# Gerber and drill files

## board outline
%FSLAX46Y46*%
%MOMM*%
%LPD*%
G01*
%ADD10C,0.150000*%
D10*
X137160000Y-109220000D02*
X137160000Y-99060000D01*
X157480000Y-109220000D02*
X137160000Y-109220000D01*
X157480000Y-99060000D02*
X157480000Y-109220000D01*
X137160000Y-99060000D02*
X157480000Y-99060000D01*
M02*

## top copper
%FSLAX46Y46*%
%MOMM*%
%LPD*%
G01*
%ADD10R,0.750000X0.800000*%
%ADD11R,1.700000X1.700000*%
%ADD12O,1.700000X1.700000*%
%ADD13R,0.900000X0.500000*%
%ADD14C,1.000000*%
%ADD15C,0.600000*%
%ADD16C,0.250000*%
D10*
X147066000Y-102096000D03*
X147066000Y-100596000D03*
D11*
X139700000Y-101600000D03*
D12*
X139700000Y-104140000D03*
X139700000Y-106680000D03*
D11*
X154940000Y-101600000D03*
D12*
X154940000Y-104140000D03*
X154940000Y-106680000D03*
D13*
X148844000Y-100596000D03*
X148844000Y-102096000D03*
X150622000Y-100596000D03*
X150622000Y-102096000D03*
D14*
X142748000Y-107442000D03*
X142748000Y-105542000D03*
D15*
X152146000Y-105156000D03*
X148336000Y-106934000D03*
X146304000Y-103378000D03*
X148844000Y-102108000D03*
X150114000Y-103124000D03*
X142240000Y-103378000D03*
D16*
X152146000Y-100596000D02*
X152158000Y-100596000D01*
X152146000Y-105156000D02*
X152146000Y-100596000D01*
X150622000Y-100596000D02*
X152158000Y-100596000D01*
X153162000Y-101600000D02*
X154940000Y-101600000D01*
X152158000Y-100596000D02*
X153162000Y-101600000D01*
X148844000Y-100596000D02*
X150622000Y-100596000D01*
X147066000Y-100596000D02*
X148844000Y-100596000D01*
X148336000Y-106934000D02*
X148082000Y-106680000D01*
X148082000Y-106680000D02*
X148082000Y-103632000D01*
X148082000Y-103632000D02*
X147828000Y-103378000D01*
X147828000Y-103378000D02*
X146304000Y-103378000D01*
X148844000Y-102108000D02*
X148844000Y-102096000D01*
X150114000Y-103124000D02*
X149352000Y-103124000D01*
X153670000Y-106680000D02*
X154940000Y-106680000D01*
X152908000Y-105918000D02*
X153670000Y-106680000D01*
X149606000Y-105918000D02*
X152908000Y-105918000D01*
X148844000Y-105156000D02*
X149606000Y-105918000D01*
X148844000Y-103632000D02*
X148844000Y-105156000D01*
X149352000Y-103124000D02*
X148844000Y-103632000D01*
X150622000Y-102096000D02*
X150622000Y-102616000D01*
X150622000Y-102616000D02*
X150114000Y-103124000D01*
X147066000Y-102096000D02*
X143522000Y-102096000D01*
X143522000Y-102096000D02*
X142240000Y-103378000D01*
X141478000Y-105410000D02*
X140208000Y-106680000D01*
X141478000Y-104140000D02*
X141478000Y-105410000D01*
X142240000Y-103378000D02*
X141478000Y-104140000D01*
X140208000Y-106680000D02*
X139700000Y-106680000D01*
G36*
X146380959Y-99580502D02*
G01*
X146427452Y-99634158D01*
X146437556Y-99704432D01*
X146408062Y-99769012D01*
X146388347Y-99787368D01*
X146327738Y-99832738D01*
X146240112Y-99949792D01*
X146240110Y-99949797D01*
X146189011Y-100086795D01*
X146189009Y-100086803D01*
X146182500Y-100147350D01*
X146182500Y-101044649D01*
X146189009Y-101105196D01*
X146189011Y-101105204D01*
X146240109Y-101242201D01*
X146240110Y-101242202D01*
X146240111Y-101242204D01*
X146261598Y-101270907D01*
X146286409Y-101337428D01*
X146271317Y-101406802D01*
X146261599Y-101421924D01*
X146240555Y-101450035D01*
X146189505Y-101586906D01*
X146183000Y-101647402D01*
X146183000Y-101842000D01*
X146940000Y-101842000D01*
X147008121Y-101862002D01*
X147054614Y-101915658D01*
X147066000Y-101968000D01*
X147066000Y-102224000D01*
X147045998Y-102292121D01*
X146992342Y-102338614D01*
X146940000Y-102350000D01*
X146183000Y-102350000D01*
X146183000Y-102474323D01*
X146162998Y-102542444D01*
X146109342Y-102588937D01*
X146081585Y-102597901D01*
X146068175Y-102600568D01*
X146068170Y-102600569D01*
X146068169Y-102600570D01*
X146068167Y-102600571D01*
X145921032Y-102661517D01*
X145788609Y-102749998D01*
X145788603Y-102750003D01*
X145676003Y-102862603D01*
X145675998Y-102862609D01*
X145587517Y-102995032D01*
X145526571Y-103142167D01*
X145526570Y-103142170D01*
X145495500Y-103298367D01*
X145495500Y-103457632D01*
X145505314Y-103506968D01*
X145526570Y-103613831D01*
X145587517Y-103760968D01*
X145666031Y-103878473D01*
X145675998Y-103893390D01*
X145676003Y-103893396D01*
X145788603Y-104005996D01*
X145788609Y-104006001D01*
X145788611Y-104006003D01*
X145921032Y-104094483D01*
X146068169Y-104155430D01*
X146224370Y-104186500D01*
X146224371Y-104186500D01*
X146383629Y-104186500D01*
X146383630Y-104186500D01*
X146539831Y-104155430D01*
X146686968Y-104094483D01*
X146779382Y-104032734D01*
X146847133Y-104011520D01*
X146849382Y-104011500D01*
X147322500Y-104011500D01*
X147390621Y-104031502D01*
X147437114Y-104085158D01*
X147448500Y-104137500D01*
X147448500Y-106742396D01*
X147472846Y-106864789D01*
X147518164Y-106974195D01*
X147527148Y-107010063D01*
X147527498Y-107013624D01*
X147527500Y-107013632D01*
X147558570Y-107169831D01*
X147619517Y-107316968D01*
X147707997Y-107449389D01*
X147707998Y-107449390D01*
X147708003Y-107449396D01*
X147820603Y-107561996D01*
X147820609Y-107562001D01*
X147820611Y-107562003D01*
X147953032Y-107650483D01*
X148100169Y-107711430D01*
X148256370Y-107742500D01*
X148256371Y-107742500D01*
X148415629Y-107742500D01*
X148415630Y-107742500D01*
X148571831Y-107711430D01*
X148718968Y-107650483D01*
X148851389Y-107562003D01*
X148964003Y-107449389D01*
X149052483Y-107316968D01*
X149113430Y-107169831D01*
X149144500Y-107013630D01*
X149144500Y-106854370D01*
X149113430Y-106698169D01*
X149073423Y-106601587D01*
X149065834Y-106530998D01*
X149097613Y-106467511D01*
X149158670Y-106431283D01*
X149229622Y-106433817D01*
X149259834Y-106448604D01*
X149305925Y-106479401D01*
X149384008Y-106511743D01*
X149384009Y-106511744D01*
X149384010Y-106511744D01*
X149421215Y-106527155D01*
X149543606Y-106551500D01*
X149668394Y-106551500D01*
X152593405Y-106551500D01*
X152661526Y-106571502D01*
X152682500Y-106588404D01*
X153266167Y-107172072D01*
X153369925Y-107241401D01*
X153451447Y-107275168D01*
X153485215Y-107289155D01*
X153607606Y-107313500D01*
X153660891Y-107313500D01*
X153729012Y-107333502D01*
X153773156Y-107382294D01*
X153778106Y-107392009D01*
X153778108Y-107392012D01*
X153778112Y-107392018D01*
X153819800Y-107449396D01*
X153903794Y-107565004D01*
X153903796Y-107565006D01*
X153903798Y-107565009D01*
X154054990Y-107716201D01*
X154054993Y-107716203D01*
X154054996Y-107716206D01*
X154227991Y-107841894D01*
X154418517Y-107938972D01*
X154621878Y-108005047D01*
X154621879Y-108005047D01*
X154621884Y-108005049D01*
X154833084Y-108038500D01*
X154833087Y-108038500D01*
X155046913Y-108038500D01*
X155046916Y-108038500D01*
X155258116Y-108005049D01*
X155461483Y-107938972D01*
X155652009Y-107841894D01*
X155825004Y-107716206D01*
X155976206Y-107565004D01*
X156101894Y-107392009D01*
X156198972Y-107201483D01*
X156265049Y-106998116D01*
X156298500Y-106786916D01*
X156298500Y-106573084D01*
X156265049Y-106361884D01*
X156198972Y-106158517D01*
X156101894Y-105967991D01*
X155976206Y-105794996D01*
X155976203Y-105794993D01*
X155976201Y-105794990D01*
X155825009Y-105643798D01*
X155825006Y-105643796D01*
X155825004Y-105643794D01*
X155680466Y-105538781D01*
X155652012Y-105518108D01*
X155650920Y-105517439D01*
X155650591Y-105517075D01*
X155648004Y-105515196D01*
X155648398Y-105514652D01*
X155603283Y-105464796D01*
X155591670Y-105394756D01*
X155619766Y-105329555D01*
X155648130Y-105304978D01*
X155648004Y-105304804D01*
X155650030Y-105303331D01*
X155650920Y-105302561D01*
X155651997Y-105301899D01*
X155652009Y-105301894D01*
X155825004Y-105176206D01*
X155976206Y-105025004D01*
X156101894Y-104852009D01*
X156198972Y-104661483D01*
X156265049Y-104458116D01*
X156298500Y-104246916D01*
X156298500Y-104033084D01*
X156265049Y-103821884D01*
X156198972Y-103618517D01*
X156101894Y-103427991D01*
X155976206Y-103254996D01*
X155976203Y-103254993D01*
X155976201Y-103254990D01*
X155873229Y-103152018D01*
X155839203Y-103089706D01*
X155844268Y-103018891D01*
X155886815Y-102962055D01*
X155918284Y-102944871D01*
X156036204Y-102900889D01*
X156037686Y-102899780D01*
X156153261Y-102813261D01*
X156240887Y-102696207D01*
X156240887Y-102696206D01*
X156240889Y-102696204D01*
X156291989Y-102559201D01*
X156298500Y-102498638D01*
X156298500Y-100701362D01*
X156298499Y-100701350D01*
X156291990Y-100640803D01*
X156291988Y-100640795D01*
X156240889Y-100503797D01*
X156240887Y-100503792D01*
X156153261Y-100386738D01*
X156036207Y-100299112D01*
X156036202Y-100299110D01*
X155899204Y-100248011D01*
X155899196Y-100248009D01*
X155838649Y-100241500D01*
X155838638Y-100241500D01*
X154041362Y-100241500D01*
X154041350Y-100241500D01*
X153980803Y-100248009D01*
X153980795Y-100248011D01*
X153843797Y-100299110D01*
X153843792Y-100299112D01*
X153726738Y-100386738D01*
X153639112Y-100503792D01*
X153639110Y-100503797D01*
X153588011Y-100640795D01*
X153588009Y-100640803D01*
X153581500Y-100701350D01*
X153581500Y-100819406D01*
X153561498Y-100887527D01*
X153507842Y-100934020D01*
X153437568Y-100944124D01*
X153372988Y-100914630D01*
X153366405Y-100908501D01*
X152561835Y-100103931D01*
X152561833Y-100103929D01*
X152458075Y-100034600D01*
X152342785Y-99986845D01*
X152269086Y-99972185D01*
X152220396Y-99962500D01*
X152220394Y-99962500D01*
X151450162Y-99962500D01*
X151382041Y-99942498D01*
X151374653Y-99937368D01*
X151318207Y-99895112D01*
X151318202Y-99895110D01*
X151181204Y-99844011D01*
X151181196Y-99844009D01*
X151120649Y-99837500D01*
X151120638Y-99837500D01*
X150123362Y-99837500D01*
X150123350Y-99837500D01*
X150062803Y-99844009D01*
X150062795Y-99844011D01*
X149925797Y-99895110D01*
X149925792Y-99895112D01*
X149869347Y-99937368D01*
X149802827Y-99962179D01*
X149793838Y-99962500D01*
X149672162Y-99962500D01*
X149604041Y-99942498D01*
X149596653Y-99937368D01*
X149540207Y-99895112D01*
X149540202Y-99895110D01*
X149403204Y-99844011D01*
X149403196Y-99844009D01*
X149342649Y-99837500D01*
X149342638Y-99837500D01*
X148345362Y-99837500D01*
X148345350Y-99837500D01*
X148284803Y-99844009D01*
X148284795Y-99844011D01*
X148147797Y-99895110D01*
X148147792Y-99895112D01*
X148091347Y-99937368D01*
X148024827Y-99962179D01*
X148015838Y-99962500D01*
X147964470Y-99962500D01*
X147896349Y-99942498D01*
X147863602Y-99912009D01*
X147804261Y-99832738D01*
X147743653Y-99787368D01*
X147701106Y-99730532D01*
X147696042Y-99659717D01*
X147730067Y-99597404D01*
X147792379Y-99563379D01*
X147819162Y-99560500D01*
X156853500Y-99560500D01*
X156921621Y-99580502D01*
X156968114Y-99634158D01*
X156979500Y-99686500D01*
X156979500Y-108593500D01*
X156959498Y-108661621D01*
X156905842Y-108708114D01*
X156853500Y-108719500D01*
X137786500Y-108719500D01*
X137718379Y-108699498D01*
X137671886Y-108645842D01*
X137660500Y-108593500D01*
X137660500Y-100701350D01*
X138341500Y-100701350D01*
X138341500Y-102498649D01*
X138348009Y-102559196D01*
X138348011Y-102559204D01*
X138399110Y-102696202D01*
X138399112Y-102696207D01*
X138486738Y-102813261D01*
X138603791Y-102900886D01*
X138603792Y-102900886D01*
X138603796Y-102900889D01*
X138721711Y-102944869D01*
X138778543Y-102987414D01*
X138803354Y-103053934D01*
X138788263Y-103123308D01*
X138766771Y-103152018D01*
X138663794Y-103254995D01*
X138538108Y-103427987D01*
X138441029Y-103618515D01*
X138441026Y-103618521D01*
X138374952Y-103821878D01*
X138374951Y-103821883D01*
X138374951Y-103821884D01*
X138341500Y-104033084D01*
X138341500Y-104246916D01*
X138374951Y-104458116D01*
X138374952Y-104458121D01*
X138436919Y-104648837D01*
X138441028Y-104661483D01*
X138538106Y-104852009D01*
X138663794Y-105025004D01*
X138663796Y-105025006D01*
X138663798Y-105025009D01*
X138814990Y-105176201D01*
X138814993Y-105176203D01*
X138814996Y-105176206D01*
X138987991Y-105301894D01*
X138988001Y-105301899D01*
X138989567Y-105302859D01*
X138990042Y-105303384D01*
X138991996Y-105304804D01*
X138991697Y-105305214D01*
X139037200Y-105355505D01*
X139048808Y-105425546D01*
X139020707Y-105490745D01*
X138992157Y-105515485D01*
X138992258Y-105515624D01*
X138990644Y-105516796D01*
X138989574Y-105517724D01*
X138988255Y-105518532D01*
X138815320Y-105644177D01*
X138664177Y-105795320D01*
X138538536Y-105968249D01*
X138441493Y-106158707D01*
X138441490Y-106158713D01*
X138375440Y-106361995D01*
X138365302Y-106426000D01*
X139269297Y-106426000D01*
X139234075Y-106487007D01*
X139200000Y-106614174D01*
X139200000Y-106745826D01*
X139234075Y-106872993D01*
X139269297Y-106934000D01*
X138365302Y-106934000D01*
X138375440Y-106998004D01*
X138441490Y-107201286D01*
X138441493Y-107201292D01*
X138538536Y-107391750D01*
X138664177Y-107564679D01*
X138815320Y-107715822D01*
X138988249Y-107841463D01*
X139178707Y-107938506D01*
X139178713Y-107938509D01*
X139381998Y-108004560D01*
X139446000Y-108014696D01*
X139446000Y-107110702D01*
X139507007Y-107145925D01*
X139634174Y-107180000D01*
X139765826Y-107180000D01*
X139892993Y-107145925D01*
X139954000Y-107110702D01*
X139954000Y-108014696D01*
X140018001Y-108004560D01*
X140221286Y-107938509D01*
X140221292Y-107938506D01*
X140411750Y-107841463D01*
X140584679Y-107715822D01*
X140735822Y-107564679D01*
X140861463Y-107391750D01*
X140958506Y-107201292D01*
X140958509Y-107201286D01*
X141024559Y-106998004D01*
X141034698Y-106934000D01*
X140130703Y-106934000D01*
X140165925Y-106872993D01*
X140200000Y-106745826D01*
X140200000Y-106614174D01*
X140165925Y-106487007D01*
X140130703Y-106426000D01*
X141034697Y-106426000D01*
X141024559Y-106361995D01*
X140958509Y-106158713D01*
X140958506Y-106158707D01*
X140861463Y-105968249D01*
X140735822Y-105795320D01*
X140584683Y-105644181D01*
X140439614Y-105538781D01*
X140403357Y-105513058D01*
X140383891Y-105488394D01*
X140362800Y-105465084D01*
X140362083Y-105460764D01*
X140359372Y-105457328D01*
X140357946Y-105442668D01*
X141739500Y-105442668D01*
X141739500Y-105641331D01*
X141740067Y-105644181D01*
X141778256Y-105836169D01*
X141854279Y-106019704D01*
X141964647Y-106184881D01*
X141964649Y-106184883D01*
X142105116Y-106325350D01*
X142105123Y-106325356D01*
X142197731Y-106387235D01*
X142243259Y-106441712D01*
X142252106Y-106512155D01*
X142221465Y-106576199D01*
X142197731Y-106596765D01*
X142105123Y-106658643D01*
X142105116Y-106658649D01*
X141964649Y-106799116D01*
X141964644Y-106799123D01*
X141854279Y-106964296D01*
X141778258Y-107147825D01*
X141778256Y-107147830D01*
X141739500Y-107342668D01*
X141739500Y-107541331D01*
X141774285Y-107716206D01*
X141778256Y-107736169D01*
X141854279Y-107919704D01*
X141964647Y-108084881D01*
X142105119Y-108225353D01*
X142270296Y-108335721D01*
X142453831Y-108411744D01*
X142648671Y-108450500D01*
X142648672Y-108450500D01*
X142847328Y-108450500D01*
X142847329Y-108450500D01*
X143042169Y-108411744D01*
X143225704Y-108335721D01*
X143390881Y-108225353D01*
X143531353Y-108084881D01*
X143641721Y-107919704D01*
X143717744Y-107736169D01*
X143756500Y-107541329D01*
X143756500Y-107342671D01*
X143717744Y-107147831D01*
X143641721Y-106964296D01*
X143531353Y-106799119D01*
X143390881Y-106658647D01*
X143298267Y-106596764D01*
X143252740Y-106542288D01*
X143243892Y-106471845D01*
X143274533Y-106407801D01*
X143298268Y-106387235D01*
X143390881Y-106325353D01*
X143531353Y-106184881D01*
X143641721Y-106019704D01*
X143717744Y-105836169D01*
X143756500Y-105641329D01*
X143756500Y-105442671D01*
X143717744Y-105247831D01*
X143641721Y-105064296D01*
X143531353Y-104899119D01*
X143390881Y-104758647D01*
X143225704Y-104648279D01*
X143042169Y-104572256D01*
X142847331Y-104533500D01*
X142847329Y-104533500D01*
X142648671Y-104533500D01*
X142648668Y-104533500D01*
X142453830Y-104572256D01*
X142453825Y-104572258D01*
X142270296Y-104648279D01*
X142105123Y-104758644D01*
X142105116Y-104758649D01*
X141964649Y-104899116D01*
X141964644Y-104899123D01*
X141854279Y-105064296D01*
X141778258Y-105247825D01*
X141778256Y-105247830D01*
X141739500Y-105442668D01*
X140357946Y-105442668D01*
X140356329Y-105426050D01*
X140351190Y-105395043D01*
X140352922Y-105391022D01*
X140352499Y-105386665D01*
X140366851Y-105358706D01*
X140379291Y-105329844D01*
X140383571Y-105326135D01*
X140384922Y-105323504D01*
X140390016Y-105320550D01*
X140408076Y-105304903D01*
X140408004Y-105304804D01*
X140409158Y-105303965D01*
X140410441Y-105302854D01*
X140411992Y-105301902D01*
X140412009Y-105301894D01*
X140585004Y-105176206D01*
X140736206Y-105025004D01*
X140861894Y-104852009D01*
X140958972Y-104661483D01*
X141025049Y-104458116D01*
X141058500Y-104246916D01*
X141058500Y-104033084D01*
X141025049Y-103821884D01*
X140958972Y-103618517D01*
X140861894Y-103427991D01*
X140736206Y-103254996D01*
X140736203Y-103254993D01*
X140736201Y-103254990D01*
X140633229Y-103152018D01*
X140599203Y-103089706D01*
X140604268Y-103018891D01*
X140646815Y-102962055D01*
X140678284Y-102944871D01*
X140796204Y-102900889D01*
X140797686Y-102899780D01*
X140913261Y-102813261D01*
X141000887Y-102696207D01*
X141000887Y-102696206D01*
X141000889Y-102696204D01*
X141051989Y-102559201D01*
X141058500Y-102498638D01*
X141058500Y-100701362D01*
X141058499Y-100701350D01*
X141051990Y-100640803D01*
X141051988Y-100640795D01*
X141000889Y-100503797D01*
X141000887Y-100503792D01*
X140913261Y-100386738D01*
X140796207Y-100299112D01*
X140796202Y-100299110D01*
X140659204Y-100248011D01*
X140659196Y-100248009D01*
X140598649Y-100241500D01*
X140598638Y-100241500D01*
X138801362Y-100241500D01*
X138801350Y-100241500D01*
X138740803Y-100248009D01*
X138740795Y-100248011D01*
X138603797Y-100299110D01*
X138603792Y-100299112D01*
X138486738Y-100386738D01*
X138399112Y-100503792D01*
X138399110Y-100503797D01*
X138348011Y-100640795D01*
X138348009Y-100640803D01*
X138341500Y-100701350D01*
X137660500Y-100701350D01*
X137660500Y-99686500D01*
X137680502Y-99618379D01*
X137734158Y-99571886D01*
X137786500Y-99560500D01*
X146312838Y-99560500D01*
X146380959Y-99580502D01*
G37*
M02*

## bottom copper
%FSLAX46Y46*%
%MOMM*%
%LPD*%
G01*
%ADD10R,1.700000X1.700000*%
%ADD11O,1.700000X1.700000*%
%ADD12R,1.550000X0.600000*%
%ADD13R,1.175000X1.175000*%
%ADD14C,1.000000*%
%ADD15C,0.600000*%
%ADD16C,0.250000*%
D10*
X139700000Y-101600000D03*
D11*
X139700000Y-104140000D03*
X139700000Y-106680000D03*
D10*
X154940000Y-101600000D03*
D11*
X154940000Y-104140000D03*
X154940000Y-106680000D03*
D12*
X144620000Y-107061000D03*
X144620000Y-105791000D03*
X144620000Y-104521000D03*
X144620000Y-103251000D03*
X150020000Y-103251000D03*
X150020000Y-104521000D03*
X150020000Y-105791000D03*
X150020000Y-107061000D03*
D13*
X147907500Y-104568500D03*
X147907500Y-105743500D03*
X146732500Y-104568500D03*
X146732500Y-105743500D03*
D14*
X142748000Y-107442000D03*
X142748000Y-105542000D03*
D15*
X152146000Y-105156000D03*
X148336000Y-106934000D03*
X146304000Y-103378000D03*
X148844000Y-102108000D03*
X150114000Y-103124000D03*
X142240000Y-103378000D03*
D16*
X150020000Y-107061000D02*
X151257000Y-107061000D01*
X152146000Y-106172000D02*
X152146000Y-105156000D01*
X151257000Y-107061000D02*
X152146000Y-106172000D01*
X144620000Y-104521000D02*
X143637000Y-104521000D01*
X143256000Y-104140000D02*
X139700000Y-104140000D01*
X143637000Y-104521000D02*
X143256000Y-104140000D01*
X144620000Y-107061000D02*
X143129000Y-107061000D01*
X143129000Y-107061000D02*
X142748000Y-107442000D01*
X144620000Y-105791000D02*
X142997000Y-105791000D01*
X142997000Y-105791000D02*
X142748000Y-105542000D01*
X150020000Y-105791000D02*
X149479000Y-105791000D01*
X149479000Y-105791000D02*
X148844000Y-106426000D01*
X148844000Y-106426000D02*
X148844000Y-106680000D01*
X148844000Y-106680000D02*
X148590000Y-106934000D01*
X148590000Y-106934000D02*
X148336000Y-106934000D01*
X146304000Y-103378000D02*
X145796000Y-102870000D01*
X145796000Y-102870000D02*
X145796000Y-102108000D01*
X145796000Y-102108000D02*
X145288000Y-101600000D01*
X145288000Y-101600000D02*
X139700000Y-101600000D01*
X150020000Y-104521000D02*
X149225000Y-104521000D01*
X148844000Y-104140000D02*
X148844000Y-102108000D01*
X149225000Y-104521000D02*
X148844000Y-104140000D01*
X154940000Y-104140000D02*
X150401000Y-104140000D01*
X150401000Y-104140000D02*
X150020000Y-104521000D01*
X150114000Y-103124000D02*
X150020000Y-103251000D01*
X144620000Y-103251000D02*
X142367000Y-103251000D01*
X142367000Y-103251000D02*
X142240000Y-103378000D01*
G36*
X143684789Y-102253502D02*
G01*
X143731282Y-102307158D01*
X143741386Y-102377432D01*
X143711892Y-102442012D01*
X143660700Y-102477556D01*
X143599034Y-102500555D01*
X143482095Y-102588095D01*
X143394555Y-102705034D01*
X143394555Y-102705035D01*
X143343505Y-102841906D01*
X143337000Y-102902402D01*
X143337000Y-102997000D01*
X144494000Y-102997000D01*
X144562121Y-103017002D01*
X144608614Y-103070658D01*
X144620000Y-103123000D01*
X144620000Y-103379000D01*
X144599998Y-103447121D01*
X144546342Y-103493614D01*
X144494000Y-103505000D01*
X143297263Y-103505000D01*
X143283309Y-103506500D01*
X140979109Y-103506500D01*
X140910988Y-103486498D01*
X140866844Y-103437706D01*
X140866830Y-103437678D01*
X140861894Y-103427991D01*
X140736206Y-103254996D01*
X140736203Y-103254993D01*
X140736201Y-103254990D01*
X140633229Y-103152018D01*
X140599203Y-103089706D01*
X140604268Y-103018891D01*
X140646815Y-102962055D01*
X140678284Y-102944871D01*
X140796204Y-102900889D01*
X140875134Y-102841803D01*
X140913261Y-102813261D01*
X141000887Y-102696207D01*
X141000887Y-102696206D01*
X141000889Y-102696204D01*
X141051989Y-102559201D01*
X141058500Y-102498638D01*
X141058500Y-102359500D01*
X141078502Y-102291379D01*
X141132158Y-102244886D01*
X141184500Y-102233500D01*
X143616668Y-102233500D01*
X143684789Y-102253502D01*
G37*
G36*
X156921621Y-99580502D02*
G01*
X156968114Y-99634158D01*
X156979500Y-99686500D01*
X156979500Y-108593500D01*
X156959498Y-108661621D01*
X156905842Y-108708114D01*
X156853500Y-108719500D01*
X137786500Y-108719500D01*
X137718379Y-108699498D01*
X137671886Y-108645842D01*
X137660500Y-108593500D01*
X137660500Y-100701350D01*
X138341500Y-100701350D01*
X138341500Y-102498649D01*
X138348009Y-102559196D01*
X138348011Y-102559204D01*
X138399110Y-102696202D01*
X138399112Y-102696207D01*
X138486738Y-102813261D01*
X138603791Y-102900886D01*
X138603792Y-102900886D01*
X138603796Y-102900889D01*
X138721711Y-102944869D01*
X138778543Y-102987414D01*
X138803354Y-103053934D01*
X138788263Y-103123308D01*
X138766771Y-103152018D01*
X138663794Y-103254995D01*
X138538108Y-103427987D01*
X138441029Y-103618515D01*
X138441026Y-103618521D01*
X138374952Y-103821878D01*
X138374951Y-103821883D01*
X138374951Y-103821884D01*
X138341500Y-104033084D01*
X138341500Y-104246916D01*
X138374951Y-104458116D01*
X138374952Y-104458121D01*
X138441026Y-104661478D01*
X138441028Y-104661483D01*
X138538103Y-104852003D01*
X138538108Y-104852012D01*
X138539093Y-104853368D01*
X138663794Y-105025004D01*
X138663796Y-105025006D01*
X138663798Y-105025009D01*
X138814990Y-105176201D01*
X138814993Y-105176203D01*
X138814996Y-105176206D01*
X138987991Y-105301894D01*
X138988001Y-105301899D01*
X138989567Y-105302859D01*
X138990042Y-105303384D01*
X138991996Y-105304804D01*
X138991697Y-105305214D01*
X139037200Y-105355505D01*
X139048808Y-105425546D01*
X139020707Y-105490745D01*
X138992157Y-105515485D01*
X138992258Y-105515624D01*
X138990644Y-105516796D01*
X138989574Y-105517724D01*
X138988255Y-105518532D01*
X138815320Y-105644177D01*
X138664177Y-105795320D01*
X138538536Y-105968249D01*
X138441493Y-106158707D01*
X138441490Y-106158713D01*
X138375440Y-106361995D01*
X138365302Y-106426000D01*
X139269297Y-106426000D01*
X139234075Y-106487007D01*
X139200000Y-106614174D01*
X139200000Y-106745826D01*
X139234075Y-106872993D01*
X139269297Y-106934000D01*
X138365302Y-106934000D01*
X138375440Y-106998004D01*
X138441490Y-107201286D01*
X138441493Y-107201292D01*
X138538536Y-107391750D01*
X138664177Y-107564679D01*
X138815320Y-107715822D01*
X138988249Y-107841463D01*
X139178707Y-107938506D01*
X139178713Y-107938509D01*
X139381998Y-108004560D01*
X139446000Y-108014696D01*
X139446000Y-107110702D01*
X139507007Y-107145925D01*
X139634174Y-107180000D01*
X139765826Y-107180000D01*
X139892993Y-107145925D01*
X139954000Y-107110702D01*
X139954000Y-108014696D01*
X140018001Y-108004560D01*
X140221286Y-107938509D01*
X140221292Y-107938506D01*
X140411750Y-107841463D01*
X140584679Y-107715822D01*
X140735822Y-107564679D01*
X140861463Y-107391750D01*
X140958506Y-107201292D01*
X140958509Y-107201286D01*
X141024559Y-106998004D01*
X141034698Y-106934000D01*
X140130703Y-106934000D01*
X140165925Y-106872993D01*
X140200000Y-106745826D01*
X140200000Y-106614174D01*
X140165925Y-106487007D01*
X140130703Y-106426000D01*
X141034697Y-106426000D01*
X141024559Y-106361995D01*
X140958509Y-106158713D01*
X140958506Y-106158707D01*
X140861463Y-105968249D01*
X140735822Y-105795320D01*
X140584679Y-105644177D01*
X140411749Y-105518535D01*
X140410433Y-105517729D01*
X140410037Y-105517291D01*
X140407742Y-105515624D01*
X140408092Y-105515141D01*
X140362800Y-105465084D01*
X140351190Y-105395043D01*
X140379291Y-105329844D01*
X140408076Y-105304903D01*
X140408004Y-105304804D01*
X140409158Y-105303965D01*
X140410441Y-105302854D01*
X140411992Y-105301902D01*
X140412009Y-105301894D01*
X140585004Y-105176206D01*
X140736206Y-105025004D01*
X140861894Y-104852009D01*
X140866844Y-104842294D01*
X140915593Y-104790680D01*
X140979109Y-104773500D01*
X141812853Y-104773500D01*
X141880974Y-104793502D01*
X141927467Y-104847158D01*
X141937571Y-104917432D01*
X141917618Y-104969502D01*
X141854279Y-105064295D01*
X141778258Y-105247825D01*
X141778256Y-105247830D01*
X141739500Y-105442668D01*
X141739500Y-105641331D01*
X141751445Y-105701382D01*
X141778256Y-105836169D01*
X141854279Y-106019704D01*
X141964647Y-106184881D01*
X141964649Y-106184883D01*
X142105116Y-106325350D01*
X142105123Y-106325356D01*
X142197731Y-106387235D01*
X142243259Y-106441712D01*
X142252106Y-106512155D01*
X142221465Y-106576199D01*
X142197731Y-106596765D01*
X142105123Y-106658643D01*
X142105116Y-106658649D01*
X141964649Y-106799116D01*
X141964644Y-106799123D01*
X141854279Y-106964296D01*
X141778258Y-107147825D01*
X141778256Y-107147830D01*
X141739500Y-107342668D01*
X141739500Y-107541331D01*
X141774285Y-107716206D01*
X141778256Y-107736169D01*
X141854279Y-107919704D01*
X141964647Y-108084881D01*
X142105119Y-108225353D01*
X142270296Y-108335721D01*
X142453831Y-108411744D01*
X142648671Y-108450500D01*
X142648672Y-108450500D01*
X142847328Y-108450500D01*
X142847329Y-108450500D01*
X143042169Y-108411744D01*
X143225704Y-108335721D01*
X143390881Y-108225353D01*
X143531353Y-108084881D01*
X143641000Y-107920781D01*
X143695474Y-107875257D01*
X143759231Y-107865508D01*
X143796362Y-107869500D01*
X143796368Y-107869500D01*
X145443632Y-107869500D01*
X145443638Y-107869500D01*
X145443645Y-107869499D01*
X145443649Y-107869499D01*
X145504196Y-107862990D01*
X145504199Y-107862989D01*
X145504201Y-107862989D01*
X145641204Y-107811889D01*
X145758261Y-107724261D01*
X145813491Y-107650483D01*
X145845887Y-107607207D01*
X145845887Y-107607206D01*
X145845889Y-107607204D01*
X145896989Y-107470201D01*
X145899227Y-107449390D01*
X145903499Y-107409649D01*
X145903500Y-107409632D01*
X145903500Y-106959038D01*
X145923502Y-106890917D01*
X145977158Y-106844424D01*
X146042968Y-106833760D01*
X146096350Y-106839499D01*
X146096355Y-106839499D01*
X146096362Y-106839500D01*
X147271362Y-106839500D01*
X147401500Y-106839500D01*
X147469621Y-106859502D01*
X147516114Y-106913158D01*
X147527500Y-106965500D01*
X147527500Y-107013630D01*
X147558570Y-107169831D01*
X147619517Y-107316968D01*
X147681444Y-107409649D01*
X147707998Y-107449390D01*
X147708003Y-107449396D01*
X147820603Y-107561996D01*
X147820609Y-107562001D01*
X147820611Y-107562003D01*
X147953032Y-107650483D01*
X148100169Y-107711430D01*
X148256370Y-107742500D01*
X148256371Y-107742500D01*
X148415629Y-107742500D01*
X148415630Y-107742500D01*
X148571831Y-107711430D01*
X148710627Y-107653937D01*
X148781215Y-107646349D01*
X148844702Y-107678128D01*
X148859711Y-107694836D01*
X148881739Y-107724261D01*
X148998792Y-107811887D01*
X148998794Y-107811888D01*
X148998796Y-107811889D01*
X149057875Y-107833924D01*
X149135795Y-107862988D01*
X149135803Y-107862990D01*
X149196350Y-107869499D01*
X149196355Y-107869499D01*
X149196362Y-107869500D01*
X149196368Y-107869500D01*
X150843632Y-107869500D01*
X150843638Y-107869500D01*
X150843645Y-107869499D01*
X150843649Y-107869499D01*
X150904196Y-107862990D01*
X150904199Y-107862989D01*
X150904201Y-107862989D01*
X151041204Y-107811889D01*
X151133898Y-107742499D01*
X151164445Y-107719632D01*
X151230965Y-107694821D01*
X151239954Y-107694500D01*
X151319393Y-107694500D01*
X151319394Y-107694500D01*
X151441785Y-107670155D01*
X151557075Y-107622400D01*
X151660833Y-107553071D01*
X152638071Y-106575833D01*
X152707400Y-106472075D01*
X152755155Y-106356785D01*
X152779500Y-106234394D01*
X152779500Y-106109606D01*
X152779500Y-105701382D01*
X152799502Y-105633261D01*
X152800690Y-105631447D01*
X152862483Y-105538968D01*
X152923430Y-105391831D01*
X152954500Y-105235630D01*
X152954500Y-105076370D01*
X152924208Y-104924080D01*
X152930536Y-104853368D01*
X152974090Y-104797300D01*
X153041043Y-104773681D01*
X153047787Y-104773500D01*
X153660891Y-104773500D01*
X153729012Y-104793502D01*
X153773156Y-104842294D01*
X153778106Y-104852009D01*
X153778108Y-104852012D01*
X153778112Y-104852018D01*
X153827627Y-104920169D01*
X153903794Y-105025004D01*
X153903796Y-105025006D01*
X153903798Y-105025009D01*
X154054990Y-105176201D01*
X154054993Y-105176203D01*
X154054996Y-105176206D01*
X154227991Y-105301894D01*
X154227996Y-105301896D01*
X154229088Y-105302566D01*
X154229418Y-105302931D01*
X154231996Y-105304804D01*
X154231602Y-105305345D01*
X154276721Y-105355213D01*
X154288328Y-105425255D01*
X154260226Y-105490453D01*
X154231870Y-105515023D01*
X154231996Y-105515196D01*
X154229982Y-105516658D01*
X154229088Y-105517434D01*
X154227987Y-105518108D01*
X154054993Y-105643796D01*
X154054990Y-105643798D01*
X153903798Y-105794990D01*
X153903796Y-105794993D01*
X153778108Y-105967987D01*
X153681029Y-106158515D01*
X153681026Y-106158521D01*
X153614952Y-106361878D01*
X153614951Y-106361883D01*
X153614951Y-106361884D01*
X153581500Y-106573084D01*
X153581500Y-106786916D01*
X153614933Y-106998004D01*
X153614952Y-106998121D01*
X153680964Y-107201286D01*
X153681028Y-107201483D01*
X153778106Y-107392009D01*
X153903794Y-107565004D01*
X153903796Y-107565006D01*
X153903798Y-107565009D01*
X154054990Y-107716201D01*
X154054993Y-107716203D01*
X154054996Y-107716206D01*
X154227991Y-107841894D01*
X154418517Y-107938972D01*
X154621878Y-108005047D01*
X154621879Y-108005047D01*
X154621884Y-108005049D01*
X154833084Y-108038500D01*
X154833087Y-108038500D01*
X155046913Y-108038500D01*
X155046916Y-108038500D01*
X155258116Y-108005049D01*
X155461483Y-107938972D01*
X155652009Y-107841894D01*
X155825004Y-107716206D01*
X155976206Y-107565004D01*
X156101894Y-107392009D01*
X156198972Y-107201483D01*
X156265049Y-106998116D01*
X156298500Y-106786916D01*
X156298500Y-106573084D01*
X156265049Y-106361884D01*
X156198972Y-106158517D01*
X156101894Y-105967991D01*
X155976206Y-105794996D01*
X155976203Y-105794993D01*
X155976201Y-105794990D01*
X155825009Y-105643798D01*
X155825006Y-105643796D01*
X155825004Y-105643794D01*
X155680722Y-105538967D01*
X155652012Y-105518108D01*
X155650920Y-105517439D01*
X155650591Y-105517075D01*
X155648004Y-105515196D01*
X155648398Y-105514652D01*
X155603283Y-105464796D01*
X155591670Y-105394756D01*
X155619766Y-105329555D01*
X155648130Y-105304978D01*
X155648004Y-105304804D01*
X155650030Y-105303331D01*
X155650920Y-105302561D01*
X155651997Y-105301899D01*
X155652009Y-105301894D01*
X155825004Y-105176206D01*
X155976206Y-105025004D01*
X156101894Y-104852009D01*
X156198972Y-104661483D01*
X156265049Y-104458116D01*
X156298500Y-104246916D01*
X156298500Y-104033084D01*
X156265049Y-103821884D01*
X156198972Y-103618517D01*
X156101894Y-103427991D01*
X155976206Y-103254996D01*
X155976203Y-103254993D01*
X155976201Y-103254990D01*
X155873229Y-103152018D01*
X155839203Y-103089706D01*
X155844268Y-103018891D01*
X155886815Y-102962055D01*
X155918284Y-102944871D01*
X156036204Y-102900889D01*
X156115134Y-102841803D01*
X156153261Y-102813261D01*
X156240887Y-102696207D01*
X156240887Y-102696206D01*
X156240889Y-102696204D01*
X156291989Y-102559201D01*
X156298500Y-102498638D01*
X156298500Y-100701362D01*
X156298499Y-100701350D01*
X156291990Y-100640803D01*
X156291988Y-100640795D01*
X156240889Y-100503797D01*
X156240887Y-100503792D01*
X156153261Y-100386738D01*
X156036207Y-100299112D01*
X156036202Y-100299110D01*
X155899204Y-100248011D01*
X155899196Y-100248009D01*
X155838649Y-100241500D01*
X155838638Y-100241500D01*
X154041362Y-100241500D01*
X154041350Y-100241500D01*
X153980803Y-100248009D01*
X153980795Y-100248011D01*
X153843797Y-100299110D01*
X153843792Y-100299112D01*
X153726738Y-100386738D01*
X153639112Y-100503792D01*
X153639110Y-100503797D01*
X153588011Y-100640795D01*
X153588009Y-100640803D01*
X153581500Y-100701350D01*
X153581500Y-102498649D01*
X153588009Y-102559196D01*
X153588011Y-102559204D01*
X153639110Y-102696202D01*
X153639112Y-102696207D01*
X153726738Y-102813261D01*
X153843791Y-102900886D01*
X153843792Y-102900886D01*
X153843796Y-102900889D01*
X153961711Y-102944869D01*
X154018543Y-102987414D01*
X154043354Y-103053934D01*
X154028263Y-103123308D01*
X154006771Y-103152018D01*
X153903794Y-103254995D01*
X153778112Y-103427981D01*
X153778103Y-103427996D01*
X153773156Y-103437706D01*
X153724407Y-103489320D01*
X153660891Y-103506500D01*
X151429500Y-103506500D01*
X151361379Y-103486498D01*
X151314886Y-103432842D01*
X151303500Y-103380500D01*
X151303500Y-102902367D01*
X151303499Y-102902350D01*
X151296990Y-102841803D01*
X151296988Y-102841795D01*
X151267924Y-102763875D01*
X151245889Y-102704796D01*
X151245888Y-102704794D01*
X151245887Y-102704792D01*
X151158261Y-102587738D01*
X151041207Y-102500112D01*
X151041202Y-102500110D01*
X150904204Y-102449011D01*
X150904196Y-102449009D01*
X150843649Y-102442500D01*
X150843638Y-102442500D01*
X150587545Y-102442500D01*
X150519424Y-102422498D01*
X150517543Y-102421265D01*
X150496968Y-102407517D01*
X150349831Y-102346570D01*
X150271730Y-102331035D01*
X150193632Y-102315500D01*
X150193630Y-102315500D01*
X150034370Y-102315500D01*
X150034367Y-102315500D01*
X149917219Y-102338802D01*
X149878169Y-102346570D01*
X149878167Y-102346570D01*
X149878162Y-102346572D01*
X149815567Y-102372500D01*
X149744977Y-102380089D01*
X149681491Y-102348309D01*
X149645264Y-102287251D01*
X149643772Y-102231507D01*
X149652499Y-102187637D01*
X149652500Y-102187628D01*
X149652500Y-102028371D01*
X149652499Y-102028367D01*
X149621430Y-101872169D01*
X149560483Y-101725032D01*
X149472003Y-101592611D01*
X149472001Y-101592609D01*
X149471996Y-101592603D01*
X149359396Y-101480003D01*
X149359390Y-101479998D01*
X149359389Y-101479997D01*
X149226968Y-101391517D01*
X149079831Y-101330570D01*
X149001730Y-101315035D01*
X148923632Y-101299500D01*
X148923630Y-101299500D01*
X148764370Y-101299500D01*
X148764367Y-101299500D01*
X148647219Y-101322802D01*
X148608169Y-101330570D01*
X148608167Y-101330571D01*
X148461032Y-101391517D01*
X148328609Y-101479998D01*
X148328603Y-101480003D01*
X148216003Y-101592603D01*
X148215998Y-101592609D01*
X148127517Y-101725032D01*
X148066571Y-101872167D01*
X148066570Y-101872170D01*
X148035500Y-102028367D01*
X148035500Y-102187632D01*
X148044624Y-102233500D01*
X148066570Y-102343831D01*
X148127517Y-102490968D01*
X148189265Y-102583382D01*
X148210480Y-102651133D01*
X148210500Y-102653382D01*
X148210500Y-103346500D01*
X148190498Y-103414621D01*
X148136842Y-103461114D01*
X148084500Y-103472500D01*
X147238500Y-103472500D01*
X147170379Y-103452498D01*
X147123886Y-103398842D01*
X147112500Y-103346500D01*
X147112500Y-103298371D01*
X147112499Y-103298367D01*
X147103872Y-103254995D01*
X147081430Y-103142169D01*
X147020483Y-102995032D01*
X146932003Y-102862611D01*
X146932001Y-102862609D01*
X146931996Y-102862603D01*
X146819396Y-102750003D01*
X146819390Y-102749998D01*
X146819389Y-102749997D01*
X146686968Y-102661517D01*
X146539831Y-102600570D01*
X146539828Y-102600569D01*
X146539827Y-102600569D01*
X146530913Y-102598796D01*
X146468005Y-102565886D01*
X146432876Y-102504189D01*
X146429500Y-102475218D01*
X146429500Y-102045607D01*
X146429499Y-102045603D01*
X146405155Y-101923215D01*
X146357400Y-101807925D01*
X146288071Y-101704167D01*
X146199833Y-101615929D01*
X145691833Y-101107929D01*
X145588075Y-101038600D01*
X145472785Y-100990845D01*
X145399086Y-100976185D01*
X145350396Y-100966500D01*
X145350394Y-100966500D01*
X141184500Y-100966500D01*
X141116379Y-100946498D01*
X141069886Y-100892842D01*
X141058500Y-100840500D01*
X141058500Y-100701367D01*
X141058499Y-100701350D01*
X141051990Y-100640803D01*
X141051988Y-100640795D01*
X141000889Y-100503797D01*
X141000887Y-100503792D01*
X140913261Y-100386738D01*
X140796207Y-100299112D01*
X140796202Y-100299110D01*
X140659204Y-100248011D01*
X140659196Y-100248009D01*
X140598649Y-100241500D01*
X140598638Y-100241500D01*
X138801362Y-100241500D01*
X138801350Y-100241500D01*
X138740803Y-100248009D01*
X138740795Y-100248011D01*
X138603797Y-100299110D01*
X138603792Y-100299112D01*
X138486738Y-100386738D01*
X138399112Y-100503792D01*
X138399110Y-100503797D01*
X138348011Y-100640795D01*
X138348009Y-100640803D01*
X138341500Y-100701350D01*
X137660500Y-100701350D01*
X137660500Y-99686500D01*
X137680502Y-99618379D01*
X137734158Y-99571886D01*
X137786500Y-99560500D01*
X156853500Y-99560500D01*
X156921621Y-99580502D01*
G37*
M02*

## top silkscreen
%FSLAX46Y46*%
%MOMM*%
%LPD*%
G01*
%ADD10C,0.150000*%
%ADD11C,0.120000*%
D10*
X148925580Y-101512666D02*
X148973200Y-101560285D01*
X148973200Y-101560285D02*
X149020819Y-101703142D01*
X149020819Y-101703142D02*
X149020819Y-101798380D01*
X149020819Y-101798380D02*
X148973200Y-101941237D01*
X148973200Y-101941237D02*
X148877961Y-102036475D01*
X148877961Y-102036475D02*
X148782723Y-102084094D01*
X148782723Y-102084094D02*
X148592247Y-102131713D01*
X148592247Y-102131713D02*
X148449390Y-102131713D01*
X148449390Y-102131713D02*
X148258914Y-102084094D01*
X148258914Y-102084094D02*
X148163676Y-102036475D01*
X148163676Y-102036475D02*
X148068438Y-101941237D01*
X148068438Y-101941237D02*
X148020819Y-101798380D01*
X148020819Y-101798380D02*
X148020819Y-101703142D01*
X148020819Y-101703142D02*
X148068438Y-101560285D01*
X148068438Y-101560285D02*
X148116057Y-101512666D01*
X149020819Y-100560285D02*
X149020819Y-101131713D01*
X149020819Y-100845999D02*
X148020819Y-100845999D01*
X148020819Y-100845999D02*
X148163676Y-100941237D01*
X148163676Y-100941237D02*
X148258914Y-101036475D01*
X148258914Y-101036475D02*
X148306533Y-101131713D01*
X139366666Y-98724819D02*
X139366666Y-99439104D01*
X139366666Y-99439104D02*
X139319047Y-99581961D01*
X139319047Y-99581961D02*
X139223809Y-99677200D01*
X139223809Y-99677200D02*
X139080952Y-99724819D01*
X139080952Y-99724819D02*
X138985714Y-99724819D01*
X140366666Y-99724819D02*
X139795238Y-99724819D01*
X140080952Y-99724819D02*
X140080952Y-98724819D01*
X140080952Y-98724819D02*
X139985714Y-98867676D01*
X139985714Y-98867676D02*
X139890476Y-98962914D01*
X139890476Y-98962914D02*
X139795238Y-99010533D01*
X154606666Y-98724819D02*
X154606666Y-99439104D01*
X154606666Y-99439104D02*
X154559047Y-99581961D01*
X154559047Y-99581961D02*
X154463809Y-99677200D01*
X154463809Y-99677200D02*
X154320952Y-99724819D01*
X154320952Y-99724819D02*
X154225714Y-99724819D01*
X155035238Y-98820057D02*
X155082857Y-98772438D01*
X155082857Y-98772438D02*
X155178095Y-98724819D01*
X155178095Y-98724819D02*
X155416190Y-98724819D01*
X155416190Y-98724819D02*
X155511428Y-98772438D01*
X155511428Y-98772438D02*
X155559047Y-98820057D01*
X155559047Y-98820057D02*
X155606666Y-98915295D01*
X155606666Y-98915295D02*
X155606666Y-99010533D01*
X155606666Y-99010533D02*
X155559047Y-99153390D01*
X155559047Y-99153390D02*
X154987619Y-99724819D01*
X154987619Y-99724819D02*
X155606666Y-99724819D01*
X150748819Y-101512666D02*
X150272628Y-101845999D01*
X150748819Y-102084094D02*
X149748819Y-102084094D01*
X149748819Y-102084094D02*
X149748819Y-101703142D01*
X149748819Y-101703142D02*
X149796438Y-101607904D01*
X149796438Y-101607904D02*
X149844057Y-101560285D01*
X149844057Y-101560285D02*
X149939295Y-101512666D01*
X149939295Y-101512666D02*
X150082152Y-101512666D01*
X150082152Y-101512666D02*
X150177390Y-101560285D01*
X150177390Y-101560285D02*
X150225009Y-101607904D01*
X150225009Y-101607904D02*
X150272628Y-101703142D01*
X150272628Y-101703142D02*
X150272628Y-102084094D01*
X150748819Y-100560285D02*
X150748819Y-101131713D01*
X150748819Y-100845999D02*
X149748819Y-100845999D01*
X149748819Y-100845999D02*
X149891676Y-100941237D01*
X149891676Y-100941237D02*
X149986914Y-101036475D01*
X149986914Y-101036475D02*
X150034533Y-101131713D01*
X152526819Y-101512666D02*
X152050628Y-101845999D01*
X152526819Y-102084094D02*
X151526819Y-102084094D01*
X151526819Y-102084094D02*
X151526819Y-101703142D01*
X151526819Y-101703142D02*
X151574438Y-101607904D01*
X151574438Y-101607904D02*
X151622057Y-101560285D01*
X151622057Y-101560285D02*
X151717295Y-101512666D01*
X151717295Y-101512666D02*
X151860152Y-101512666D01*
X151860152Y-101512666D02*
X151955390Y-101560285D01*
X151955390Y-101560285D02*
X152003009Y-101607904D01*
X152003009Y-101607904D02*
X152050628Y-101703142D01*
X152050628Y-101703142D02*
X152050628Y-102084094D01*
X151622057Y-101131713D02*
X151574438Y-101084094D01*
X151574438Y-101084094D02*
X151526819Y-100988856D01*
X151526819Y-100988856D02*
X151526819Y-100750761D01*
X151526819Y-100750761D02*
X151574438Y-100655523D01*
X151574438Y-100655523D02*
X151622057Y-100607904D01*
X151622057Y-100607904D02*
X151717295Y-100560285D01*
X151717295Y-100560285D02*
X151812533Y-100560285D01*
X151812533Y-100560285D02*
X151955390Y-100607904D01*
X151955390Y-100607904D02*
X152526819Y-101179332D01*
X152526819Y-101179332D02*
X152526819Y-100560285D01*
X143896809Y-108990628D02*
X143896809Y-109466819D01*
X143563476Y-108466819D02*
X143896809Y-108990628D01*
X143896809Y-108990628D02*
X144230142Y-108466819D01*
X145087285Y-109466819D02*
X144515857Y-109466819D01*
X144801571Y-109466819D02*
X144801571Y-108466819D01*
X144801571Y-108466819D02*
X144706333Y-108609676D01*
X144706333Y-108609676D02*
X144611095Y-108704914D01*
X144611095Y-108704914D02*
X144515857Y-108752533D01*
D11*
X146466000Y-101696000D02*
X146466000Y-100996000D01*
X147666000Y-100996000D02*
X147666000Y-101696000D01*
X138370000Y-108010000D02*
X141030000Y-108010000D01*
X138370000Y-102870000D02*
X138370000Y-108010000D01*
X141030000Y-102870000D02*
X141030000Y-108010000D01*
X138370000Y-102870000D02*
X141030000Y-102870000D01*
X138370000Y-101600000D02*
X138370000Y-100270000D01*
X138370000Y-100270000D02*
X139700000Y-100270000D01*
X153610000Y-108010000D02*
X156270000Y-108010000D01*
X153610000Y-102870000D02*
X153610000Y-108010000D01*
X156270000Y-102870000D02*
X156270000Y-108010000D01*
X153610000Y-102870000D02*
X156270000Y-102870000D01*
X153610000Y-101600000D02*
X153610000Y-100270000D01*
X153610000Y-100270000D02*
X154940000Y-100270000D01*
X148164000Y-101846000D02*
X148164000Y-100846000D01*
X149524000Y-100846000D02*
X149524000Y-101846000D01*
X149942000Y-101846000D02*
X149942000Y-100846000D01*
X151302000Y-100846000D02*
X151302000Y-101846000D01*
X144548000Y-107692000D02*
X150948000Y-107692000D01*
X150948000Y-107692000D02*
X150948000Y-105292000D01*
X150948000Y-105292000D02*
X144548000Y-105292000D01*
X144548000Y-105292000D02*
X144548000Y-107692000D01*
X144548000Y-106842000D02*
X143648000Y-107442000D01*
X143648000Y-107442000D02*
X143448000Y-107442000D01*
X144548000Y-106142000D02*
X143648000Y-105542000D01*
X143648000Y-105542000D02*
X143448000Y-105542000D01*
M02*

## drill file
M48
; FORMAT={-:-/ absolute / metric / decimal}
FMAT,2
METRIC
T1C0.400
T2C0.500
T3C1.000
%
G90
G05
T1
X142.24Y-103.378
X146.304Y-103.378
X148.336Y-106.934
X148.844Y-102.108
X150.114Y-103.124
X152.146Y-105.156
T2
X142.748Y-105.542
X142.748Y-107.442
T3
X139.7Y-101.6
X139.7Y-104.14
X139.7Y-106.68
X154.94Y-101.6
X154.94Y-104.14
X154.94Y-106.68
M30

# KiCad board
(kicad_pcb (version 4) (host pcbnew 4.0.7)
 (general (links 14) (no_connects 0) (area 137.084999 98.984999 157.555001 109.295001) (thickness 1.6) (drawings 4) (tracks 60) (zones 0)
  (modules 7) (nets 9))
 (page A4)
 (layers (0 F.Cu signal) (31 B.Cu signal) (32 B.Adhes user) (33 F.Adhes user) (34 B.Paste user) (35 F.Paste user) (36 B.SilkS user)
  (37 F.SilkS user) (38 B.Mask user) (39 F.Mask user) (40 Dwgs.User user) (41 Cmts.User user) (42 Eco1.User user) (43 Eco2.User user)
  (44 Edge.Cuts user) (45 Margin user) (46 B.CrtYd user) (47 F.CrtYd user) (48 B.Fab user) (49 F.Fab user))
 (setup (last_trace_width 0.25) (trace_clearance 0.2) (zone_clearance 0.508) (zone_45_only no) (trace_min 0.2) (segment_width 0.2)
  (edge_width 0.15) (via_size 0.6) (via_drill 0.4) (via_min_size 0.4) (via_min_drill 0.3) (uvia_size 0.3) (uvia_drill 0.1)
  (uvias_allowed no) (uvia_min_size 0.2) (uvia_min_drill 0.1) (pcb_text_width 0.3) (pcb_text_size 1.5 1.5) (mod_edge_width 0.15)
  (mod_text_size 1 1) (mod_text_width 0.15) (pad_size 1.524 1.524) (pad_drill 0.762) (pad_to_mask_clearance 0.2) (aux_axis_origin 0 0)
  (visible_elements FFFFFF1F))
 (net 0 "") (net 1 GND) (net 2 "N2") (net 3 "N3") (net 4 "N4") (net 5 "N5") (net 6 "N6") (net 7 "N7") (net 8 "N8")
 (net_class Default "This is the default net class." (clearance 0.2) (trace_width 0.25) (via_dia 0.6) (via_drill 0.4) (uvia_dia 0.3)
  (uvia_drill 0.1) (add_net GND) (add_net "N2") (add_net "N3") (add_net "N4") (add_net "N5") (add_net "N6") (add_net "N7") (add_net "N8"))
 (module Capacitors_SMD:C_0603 (layer F.Cu) (at 147.066 101.346 270)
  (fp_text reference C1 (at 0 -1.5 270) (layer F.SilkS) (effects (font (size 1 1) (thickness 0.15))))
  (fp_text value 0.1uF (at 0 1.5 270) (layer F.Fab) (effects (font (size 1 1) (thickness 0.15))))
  (fp_line (start 0.35 0.6) (end -0.35 0.6) (layer F.SilkS) (width 0.12))
  (fp_line (start -0.35 -0.6) (end 0.35 -0.6) (layer F.SilkS) (width 0.12))
  (pad 2 smd rect (at 0.75 0 270) (size 0.8 0.75) (layers F.Cu F.Paste F.Mask) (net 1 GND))
  (pad 1 smd rect (at -0.75 0 270) (size 0.8 0.75) (layers F.Cu F.Paste F.Mask) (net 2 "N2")))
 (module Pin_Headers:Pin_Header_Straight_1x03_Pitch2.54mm (layer F.Cu) (at 139.7 101.6)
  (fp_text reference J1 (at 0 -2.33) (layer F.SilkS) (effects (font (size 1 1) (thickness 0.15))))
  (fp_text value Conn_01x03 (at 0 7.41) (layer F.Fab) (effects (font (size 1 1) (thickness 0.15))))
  (fp_line (start -1.33 6.41) (end 1.33 6.41) (layer F.SilkS) (width 0.12))
  (fp_line (start -1.33 1.27) (end -1.33 6.41) (layer F.SilkS) (width 0.12))
  (fp_line (start 1.33 1.27) (end 1.33 6.41) (layer F.SilkS) (width 0.12))
  (fp_line (start -1.33 1.27) (end 1.33 1.27) (layer F.SilkS) (width 0.12))
  (fp_line (start -1.33 0) (end -1.33 -1.33) (layer F.SilkS) (width 0.12))
  (fp_line (start -1.33 -1.33) (end 0 -1.33) (layer F.SilkS) (width 0.12))
  (pad 1 thru_hole rect (at 0 0) (size 1.7 1.7) (drill 1) (layers *.Cu *.Mask) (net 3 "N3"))
  (pad 2 thru_hole oval (at 0 2.54) (size 1.7 1.7) (drill 1) (layers *.Cu *.Mask) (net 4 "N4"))
  (pad 3 thru_hole oval (at 0 5.08) (size 1.7 1.7) (drill 1) (layers *.Cu *.Mask) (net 1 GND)))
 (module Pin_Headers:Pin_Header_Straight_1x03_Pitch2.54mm (layer F.Cu) (at 154.94 101.6)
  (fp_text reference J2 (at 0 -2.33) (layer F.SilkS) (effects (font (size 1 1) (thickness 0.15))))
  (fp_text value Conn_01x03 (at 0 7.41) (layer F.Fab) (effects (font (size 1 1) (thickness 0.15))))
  (fp_line (start -1.33 6.41) (end 1.33 6.41) (layer F.SilkS) (width 0.12))
  (fp_line (start -1.33 1.27) (end -1.33 6.41) (layer F.SilkS) (width 0.12))
  (fp_line (start 1.33 1.27) (end 1.33 6.41) (layer F.SilkS) (width 0.12))
  (fp_line (start -1.33 1.27) (end 1.33 1.27) (layer F.SilkS) (width 0.12))
  (fp_line (start -1.33 0) (end -1.33 -1.33) (layer F.SilkS) (width 0.12))
  (fp_line (start -1.33 -1.33) (end 0 -1.33) (layer F.SilkS) (width 0.12))
  (pad 1 thru_hole rect (at 0 0) (size 1.7 1.7) (drill 1) (layers *.Cu *.Mask) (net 2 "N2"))
  (pad 2 thru_hole oval (at 0 2.54) (size 1.7 1.7) (drill 1) (layers *.Cu *.Mask) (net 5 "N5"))
  (pad 3 thru_hole oval (at 0 5.08) (size 1.7 1.7) (drill 1) (layers *.Cu *.Mask) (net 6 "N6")))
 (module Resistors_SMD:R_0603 (layer F.Cu) (at 148.844 101.346 270)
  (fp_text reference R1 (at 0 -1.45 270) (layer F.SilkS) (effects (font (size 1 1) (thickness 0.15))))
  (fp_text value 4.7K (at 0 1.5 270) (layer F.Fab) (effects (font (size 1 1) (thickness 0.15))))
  (fp_line (start 0.5 0.68) (end -0.5 0.68) (layer F.SilkS) (width 0.12))
  (fp_line (start -0.5 -0.68) (end 0.5 -0.68) (layer F.SilkS) (width 0.12))
  (pad 1 smd rect (at -0.75 0 270) (size 0.5 0.9) (layers F.Cu F.Paste F.Mask) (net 2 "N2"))
  (pad 2 smd rect (at 0.75 0 270) (size 0.5 0.9) (layers F.Cu F.Paste F.Mask) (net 5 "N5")))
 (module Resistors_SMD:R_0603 (layer F.Cu) (at 150.622 101.346 270)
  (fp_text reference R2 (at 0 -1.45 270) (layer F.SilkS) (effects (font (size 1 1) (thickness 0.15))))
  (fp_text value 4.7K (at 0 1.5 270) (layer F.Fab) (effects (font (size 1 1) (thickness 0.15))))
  (fp_line (start 0.5 0.68) (end -0.5 0.68) (layer F.SilkS) (width 0.12))
  (fp_line (start -0.5 -0.68) (end 0.5 -0.68) (layer F.SilkS) (width 0.12))
  (pad 1 smd rect (at -0.75 0 270) (size 0.5 0.9) (layers F.Cu F.Paste F.Mask) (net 2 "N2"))
  (pad 2 smd rect (at 0.75 0 270) (size 0.5 0.9) (layers F.Cu F.Paste F.Mask) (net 6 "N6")))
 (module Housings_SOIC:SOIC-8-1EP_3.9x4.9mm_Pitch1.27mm (layer B.Cu) (at 147.32 105.156)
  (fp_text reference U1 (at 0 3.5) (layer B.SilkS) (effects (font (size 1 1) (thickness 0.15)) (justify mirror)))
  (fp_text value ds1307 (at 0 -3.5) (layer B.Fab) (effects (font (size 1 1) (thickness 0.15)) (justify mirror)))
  (pad 1 smd rect (at -2.7 1.905) (size 1.55 0.6) (layers B.Cu B.Paste B.Mask) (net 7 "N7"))
  (pad 2 smd rect (at -2.7 0.635) (size 1.55 0.6) (layers B.Cu B.Paste B.Mask) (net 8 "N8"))
  (pad 3 smd rect (at -2.7 -0.635) (size 1.55 0.6) (layers B.Cu B.Paste B.Mask) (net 4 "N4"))
  (pad 4 smd rect (at -2.7 -1.905) (size 1.55 0.6) (layers B.Cu B.Paste B.Mask) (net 1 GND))
  (pad 5 smd rect (at 2.7 -1.905) (size 1.55 0.6) (layers B.Cu B.Paste B.Mask) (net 6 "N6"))
  (pad 6 smd rect (at 2.7 -0.635) (size 1.55 0.6) (layers B.Cu B.Paste B.Mask) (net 5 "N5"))
  (pad 7 smd rect (at 2.7 0.635) (size 1.55 0.6) (layers B.Cu B.Paste B.Mask) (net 3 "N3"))
  (pad 8 smd rect (at 2.7 1.905) (size 1.55 0.6) (layers B.Cu B.Paste B.Mask) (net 2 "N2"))
  (pad 9 smd rect (at 0.5875 -0.5875) (size 1.175 1.175) (layers B.Cu B.Paste B.Mask) (solder_paste_margin_ratio -0.2))
  (pad 9 smd rect (at 0.5875 0.5875) (size 1.175 1.175) (layers B.Cu B.Paste B.Mask) (solder_paste_margin_ratio -0.2))
  (pad 9 smd rect (at -0.5875 -0.5875) (size 1.175 1.175) (layers B.Cu B.Paste B.Mask) (solder_paste_margin_ratio -0.2))
  (pad 9 smd rect (at -0.5875 0.5875) (size 1.175 1.175) (layers B.Cu B.Paste B.Mask) (solder_paste_margin_ratio -0.2)))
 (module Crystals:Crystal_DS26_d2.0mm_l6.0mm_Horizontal (layer F.Cu) (at 142.748 107.442 90)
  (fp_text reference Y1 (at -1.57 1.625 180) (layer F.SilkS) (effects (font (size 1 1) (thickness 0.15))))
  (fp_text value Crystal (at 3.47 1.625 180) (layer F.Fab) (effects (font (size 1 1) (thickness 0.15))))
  (fp_line (start -0.25 1.8) (end -0.25 8.2) (layer F.SilkS) (width 0.12))
  (fp_line (start -0.25 8.2) (end 2.15 8.2) (layer F.SilkS) (width 0.12))
  (fp_line (start 2.15 8.2) (end 2.15 1.8) (layer F.SilkS) (width 0.12))
  (fp_line (start 2.15 1.8) (end -0.25 1.8) (layer F.SilkS) (width 0.12))
  (fp_line (start 0.6 1.8) (end 0 0.9) (layer F.SilkS) (width 0.12))
  (fp_line (start 0 0.9) (end 0 0.7) (layer F.SilkS) (width 0.12))
  (fp_line (start 1.3 1.8) (end 1.9 0.9) (layer F.SilkS) (width 0.12))
  (fp_line (start 1.9 0.9) (end 1.9 0.7) (layer F.SilkS) (width 0.12))
  (pad 1 thru_hole circle (at 0 0 90) (size 1 1) (drill 0.5) (layers *.Cu *.Mask) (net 7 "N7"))
  (pad 2 thru_hole circle (at 1.9 0 90) (size 1 1) (drill 0.5) (layers *.Cu *.Mask) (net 8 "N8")))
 (gr_line (start 137.16 109.22) (end 137.16 99.06) (angle 90) (layer Edge.Cuts) (width 0.15))
 (gr_line (start 157.48 109.22) (end 137.16 109.22) (angle 90) (layer Edge.Cuts) (width 0.15))
 (gr_line (start 157.48 99.06) (end 157.48 109.22) (angle 90) (layer Edge.Cuts) (width 0.15))
 (gr_line (start 137.16 99.06) (end 157.48 99.06) (angle 90) (layer Edge.Cuts) (width 0.15))
 (segment (start 150.02 107.061) (end 151.257 107.061) (width 0.25) (layer B.Cu) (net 2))
 (segment (start 152.146 100.596) (end 152.158 100.596) (width 0.25) (layer F.Cu) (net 2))
 (segment (start 152.146 105.156) (end 152.146 100.596) (width 0.25) (layer F.Cu) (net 2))
 (via (at 152.146 105.156) (size 0.6) (drill 0.4) (layers F.Cu B.Cu) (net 2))
 (segment (start 152.146 106.172) (end 152.146 105.156) (width 0.25) (layer B.Cu) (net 2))
 (segment (start 151.257 107.061) (end 152.146 106.172) (width 0.25) (layer B.Cu) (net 2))
 (segment (start 150.622 100.596) (end 152.158 100.596) (width 0.25) (layer F.Cu) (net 2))
 (segment (start 153.162 101.6) (end 154.94 101.6) (width 0.25) (layer F.Cu) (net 2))
 (segment (start 152.158 100.596) (end 153.162 101.6) (width 0.25) (layer F.Cu) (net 2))
 (segment (start 148.844 100.596) (end 150.622 100.596) (width 0.25) (layer F.Cu) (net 2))
 (segment (start 147.066 100.596) (end 148.844 100.596) (width 0.25) (layer F.Cu) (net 2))
 (segment (start 144.62 104.521) (end 143.637 104.521) (width 0.25) (layer B.Cu) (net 4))
 (segment (start 143.256 104.14) (end 139.7 104.14) (width 0.25) (layer B.Cu) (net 4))
 (segment (start 143.637 104.521) (end 143.256 104.14) (width 0.25) (layer B.Cu) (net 4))
 (segment (start 144.62 107.061) (end 143.129 107.061) (width 0.25) (layer B.Cu) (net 7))
 (segment (start 143.129 107.061) (end 142.748 107.442) (width 0.25) (layer B.Cu) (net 7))
 (segment (start 144.62 105.791) (end 142.997 105.791) (width 0.25) (layer B.Cu) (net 8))
 (segment (start 142.997 105.791) (end 142.748 105.542) (width 0.25) (layer B.Cu) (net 8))
 (segment (start 150.02 105.791) (end 149.479 105.791) (width 0.25) (layer B.Cu) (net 3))
 (segment (start 149.479 105.791) (end 148.844 106.426) (width 0.25) (layer B.Cu) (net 3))
 (segment (start 148.844 106.426) (end 148.844 106.68) (width 0.25) (layer B.Cu) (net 3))
 (segment (start 148.844 106.68) (end 148.59 106.934) (width 0.25) (layer B.Cu) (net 3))
 (segment (start 148.59 106.934) (end 148.336 106.934) (width 0.25) (layer B.Cu) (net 3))
 (via (at 148.336 106.934) (size 0.6) (drill 0.4) (layers F.Cu B.Cu) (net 3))
 (segment (start 148.336 106.934) (end 148.082 106.68) (width 0.25) (layer F.Cu) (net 3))
 (segment (start 148.082 106.68) (end 148.082 103.632) (width 0.25) (layer F.Cu) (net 3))
 (segment (start 148.082 103.632) (end 147.828 103.378) (width 0.25) (layer F.Cu) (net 3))
 (segment (start 147.828 103.378) (end 146.304 103.378) (width 0.25) (layer F.Cu) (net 3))
 (via (at 146.304 103.378) (size 0.6) (drill 0.4) (layers F.Cu B.Cu) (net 3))
 (segment (start 146.304 103.378) (end 145.796 102.87) (width 0.25) (layer B.Cu) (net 3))
 (segment (start 145.796 102.87) (end 145.796 102.108) (width 0.25) (layer B.Cu) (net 3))
 (segment (start 145.796 102.108) (end 145.288 101.6) (width 0.25) (layer B.Cu) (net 3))
 (segment (start 145.288 101.6) (end 139.7 101.6) (width 0.25) (layer B.Cu) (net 3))
 (segment (start 150.02 104.521) (end 149.225 104.521) (width 0.25) (layer B.Cu) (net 5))
 (segment (start 148.844 102.108) (end 148.844 102.096) (width 0.25) (layer F.Cu) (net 5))
 (via (at 148.844 102.108) (size 0.6) (drill 0.4) (layers F.Cu B.Cu) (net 5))
 (segment (start 148.844 104.14) (end 148.844 102.108) (width 0.25) (layer B.Cu) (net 5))
 (segment (start 149.225 104.521) (end 148.844 104.14) (width 0.25) (layer B.Cu) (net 5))
 (segment (start 154.94 104.14) (end 150.401 104.14) (width 0.25) (layer B.Cu) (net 5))
 (segment (start 150.401 104.14) (end 150.02 104.521) (width 0.25) (layer B.Cu) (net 5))
 (segment (start 150.114 103.124) (end 149.352 103.124) (width 0.25) (layer F.Cu) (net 6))
 (segment (start 153.67 106.68) (end 154.94 106.68) (width 0.25) (layer F.Cu) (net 6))
 (segment (start 152.908 105.918) (end 153.67 106.68) (width 0.25) (layer F.Cu) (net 6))
 (segment (start 149.606 105.918) (end 152.908 105.918) (width 0.25) (layer F.Cu) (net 6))
 (segment (start 148.844 105.156) (end 149.606 105.918) (width 0.25) (layer F.Cu) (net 6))
 (segment (start 148.844 103.632) (end 148.844 105.156) (width 0.25) (layer F.Cu) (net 6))
 (segment (start 149.352 103.124) (end 148.844 103.632) (width 0.25) (layer F.Cu) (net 6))
 (segment (start 150.622 102.096) (end 150.622 102.616) (width 0.25) (layer F.Cu) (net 6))
 (segment (start 150.114 103.124) (end 150.02 103.251) (width 0.25) (layer B.Cu) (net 6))
 (via (at 150.114 103.124) (size 0.6) (drill 0.4) (layers F.Cu B.Cu) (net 6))
 (segment (start 150.622 102.616) (end 150.114 103.124) (width 0.25) (layer F.Cu) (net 6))
 (segment (start 147.066 102.096) (end 143.522 102.096) (width 0.25) (layer F.Cu) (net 1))
 (segment (start 143.522 102.096) (end 142.24 103.378) (width 0.25) (layer F.Cu) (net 1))
 (segment (start 144.62 103.251) (end 142.367 103.251) (width 0.25) (layer B.Cu) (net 1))
 (segment (start 141.478 105.41) (end 140.208 106.68) (width 0.25) (layer F.Cu) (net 1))
 (segment (start 141.478 104.14) (end 141.478 105.41) (width 0.25) (layer F.Cu) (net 1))
 (segment (start 142.24 103.378) (end 141.478 104.14) (width 0.25) (layer F.Cu) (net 1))
 (via (at 142.24 103.378) (size 0.6) (drill 0.4) (layers F.Cu B.Cu) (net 1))
 (segment (start 142.367 103.251) (end 142.24 103.378) (width 0.25) (layer B.Cu) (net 1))
 (segment (start 140.208 106.68) (end 139.7 106.68) (width 0.25) (layer F.Cu) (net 1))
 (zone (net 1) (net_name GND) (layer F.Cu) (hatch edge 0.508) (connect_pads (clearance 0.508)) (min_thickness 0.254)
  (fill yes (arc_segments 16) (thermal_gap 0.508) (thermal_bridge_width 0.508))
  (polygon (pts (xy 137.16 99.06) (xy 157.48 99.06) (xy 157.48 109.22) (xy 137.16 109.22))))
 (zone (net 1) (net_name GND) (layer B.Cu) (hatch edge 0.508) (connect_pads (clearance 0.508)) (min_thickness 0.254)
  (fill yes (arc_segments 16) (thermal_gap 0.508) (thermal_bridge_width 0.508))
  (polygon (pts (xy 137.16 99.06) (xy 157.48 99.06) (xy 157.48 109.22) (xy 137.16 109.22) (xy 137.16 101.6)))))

